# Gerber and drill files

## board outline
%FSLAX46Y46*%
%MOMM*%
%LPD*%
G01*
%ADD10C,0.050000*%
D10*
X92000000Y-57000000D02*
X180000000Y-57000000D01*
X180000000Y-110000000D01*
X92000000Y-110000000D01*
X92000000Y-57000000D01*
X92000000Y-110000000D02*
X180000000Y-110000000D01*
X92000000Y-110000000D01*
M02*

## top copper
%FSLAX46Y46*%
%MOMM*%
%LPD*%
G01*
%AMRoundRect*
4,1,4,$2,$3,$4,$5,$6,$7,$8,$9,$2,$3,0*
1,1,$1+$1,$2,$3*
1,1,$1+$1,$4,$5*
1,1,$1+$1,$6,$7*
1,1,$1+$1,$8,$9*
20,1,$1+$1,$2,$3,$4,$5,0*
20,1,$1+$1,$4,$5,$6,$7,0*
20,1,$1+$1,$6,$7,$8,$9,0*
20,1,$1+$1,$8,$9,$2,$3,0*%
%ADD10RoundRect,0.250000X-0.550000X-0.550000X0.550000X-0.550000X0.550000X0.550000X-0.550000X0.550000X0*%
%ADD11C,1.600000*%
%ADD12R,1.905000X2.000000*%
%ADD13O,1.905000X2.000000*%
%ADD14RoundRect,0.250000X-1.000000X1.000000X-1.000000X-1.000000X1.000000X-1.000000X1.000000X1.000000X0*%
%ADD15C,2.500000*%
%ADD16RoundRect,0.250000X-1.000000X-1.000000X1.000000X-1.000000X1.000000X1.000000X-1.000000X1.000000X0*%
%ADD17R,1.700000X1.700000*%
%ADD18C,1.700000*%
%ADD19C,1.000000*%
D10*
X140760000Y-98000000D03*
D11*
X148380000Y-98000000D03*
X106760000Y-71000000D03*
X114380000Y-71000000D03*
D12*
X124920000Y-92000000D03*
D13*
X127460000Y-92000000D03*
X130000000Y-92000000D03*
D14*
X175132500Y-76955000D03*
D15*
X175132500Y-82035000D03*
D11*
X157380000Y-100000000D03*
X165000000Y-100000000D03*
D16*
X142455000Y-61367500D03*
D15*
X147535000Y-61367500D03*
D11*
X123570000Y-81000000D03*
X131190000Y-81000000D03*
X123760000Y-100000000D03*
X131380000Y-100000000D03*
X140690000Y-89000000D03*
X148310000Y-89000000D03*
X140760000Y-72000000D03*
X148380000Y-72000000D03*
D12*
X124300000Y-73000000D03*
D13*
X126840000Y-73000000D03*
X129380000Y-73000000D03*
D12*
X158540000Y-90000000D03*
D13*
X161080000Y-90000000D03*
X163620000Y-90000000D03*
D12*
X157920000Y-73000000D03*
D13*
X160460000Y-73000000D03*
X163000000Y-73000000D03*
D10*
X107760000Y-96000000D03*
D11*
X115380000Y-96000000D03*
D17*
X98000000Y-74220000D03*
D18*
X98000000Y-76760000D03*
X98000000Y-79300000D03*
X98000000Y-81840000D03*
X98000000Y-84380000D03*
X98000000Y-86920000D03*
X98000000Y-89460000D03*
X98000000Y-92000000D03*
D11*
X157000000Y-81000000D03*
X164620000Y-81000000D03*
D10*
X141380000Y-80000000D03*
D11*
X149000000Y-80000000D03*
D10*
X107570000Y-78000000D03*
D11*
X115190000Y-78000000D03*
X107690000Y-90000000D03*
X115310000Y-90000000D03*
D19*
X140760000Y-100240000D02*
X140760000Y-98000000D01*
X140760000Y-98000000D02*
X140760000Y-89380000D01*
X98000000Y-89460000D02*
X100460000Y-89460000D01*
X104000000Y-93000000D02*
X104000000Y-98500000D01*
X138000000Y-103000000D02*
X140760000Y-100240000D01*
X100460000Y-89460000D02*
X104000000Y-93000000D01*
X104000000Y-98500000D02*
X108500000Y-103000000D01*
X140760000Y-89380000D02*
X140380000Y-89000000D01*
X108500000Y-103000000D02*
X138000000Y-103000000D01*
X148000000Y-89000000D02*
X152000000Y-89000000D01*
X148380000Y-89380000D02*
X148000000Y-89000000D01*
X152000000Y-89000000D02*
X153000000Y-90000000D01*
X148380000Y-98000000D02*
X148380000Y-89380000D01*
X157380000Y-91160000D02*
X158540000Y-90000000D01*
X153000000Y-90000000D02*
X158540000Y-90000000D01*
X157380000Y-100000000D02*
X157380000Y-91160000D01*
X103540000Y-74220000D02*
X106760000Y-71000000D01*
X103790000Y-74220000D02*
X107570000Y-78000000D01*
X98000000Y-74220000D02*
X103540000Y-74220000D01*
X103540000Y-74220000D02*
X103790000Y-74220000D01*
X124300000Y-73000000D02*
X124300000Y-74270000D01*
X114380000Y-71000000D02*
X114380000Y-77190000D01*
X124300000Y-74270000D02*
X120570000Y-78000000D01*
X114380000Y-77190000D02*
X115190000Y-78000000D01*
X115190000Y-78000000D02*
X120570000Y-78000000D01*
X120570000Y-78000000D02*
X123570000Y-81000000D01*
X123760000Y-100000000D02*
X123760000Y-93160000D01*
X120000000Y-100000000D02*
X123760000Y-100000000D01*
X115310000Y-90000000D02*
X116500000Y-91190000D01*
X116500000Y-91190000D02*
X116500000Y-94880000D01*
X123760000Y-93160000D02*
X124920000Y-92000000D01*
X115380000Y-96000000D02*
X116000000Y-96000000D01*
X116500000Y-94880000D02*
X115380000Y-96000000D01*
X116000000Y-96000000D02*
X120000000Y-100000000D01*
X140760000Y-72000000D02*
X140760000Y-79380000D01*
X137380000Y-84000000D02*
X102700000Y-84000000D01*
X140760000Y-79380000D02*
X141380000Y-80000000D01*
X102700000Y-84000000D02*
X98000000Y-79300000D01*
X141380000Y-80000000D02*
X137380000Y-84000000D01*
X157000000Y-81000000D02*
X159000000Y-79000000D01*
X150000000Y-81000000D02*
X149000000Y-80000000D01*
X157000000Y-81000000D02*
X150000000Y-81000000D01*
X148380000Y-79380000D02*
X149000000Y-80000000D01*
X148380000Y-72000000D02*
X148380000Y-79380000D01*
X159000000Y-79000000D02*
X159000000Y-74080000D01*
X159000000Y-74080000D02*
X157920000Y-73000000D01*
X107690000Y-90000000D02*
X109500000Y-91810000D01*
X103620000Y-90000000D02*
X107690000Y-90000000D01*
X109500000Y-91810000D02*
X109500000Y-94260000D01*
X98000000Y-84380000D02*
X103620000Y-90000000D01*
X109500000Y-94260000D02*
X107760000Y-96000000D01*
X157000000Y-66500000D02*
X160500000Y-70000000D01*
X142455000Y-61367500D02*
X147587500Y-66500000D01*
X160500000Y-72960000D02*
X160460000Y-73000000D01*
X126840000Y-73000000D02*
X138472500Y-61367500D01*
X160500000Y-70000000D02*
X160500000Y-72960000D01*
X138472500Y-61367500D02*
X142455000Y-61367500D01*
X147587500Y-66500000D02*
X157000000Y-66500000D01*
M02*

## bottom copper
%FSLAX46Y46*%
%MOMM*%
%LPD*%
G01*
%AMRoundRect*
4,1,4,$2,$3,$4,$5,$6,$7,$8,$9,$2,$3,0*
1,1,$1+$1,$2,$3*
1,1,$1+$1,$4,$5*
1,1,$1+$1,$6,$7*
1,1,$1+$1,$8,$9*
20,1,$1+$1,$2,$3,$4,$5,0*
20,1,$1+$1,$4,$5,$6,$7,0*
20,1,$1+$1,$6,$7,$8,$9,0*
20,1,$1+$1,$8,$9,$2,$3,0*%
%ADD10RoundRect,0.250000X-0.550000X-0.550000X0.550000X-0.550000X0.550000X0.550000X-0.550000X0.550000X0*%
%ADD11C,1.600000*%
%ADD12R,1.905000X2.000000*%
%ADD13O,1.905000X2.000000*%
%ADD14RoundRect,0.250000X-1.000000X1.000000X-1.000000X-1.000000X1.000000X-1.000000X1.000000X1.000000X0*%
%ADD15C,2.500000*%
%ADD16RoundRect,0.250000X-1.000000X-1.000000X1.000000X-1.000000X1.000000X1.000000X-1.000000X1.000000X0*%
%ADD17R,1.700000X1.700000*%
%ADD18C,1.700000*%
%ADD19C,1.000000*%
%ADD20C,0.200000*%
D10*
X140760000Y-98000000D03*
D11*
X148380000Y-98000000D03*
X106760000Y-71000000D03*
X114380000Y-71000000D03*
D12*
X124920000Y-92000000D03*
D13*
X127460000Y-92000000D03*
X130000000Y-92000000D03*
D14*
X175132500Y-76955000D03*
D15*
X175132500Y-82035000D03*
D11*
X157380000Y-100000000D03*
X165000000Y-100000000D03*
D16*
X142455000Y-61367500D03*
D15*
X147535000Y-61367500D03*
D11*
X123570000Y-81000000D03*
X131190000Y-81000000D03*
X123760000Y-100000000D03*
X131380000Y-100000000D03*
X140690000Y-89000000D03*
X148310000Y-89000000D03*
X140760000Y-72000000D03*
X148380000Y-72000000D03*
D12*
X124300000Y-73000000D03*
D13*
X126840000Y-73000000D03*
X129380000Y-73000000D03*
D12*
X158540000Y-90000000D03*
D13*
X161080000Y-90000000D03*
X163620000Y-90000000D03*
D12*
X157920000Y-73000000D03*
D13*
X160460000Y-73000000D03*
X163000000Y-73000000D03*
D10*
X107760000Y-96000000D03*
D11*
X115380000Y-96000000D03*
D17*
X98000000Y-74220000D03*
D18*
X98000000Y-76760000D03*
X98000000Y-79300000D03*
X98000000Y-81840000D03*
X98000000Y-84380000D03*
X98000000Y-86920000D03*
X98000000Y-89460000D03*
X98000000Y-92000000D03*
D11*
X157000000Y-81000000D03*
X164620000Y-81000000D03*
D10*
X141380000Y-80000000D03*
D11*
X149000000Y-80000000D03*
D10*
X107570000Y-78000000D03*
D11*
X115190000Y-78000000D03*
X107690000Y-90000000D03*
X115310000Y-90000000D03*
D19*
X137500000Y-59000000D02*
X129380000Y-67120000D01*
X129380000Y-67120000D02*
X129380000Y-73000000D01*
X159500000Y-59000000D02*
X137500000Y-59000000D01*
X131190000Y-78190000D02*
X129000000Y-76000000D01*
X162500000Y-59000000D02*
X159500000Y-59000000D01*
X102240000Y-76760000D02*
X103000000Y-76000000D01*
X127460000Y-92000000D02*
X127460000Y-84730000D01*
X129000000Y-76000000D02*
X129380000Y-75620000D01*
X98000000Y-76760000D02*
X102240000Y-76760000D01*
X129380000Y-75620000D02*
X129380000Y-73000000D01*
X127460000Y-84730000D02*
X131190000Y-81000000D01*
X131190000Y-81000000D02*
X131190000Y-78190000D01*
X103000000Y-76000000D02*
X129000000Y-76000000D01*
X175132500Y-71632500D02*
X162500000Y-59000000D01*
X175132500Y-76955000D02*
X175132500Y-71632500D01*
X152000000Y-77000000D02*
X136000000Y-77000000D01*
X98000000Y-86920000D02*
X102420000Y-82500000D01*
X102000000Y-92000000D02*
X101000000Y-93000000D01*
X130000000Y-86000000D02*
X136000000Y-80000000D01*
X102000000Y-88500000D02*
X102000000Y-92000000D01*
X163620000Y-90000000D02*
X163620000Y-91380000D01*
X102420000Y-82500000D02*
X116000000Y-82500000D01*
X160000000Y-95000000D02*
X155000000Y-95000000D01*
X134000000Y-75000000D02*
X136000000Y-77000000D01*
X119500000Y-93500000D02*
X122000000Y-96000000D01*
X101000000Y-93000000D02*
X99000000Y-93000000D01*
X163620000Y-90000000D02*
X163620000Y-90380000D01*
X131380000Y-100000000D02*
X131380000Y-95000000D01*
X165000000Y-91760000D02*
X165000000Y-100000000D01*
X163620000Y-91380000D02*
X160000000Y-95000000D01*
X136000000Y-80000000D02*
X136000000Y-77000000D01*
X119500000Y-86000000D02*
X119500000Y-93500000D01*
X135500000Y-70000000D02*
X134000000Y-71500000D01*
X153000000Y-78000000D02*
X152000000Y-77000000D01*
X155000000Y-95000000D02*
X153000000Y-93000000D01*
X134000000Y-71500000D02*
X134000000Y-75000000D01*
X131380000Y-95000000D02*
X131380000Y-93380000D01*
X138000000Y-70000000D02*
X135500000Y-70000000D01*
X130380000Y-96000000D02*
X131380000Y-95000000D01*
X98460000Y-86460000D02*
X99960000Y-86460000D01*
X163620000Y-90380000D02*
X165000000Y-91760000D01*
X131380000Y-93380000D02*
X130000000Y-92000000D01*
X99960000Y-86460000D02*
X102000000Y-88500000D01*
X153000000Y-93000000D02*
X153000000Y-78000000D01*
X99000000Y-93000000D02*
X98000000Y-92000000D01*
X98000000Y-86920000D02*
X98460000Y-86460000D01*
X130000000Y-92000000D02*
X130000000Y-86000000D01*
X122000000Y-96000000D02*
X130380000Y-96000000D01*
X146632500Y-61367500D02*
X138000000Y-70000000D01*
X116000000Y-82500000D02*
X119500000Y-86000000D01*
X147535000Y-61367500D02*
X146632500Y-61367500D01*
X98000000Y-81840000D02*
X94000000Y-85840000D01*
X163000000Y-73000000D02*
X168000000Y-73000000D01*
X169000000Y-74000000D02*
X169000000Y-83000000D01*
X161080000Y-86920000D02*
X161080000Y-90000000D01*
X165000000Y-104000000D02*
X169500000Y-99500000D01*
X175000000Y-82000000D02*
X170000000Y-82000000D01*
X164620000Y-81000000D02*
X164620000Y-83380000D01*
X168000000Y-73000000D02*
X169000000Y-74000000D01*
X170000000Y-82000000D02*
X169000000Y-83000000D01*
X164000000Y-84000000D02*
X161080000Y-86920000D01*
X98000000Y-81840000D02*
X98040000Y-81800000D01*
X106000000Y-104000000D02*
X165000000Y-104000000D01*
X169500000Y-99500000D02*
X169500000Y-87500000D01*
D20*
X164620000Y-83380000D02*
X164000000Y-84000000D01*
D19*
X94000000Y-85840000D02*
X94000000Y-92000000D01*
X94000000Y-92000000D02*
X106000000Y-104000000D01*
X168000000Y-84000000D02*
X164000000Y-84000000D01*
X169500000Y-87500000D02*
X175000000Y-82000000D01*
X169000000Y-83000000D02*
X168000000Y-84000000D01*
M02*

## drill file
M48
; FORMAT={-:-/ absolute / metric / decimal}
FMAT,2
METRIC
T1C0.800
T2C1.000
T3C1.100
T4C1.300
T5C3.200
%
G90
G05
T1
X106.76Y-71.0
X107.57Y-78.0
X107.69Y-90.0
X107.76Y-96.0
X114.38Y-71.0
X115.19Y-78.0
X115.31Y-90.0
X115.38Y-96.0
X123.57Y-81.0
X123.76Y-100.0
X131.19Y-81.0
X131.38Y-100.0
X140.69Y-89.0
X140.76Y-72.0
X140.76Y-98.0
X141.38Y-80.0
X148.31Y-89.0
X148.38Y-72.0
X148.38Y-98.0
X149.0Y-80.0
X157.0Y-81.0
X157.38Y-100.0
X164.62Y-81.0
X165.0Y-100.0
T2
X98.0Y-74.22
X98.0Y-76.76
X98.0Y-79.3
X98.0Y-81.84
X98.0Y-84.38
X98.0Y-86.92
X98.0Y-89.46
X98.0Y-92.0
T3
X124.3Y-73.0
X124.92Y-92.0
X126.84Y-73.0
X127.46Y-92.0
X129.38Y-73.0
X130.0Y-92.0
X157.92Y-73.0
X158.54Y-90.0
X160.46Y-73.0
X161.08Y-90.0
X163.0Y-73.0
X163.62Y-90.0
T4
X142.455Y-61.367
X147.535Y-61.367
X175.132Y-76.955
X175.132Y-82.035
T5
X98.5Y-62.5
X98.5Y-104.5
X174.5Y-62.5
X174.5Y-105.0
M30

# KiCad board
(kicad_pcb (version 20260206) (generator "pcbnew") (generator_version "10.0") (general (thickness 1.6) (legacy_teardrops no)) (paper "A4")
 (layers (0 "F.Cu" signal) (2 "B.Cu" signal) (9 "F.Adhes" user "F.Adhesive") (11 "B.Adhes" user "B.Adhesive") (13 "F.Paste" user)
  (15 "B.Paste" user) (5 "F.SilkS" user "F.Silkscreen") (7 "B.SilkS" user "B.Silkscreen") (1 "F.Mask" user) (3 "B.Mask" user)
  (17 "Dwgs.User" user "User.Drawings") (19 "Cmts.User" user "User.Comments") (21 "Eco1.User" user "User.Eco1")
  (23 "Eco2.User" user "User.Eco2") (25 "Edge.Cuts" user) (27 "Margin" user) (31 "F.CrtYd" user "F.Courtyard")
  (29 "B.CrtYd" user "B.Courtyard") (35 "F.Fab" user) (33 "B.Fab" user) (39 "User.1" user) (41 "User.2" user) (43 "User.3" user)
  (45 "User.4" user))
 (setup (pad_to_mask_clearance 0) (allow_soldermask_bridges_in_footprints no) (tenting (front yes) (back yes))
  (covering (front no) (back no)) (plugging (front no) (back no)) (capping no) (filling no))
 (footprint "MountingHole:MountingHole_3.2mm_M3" (layer "F.Cu") (at 98.5 62.5)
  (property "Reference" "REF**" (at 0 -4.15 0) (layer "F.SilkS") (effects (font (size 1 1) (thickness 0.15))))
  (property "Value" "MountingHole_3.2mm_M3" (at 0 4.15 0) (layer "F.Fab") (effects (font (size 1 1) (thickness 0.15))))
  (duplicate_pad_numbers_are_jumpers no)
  (pad "" np_thru_hole circle (at 0 0) (size 3.2 3.2) (drill 3.2) (layers "*.Cu" "*.Mask")))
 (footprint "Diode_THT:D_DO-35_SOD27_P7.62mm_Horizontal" (layer "F.Cu") (at 140.76 98)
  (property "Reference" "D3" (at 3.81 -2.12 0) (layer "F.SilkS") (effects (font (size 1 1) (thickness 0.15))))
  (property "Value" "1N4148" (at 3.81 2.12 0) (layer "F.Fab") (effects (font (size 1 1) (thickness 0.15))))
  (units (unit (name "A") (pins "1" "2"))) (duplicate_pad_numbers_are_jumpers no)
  (pad "1" thru_hole roundrect (at 0 0) (size 1.6 1.6) (drill 0.8) (layers "*.Cu" "*.Mask") (remove_unused_layers no)
   (roundrect_rratio 0.15625) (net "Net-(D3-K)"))
  (pad "2" thru_hole circle (at 7.62 0) (size 1.6 1.6) (drill 0.8) (layers "*.Cu" "*.Mask") (remove_unused_layers no) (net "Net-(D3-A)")))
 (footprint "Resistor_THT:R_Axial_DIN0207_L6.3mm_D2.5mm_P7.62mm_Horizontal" (layer "F.Cu") (at 106.76 71)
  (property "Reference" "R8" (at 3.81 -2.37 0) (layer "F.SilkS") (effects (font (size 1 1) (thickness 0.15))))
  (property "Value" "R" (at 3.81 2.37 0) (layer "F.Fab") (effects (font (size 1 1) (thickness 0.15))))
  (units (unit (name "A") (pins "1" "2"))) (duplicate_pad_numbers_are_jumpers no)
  (pad "1" thru_hole circle (at 0 0) (size 1.6 1.6) (drill 0.8) (layers "*.Cu" "*.Mask") (remove_unused_layers no) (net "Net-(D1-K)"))
  (pad "2" thru_hole circle (at 7.62 0) (size 1.6 1.6) (drill 0.8) (layers "*.Cu" "*.Mask") (remove_unused_layers no) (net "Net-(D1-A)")))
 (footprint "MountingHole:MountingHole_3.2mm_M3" (layer "F.Cu") (at 174.5 105)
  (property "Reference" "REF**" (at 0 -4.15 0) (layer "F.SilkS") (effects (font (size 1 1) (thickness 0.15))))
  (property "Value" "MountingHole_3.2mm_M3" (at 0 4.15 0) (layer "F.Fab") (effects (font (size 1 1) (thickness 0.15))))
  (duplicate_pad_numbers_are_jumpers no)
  (pad "" np_thru_hole circle (at 0 0) (size 3.2 3.2) (drill 3.2) (layers "*.Cu" "*.Mask")))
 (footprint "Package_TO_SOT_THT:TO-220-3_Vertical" (layer "F.Cu") (at 124.92 92)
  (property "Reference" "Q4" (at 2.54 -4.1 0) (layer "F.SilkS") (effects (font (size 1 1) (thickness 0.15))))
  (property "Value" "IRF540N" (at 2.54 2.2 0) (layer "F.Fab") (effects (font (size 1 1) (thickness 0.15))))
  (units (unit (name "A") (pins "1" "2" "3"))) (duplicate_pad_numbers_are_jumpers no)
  (pad "1" thru_hole rect (at 0 0) (size 1.905 2) (drill 1.1) (layers "*.Cu" "*.Mask") (remove_unused_layers no) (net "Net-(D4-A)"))
  (pad "2" thru_hole oval (at 2.54 0) (size 1.905 2) (drill 1.1) (layers "*.Cu" "*.Mask") (remove_unused_layers no) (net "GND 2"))
  (pad "3" thru_hole oval (at 5.08 0) (size 1.905 2) (drill 1.1) (layers "*.Cu" "*.Mask") (remove_unused_layers no) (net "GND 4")))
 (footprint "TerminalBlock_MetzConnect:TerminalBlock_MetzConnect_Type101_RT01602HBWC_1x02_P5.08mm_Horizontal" (layer "F.Cu")
  (at 175.1325 76.955 -90)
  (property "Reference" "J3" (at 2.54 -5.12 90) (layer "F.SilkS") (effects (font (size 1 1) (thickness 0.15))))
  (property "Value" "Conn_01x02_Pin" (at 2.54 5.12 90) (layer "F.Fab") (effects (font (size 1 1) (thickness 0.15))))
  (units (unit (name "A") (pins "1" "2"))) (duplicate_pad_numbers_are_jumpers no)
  (pad "1" thru_hole roundrect (at 0 0 270) (size 2.5 2.5) (drill 1.3) (layers "*.Cu" "*.Mask") (remove_unused_layers no)
   (roundrect_rratio 0.1) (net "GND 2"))
  (pad "2" thru_hole circle (at 5.08 0 270) (size 2.5 2.5) (drill 1.3) (layers "*.Cu" "*.Mask") (remove_unused_layers no) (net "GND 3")))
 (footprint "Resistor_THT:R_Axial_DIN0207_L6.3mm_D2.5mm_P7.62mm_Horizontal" (layer "F.Cu") (at 157.38 100)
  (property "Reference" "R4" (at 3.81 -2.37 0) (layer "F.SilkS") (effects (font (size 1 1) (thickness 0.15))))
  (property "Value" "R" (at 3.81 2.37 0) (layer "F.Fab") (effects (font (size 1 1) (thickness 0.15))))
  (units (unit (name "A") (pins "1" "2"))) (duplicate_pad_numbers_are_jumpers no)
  (pad "1" thru_hole circle (at 0 0) (size 1.6 1.6) (drill 0.8) (layers "*.Cu" "*.Mask") (remove_unused_layers no) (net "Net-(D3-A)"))
  (pad "2" thru_hole circle (at 7.62 0) (size 1.6 1.6) (drill 0.8) (layers "*.Cu" "*.Mask") (remove_unused_layers no) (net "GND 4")))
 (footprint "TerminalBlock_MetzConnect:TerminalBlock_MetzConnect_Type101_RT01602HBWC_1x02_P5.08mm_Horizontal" (layer "F.Cu")
  (at 142.455 61.3675)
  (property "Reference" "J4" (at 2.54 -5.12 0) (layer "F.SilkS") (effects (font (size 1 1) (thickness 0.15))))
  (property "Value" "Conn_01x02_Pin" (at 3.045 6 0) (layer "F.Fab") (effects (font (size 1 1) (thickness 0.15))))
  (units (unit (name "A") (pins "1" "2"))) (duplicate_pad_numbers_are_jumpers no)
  (pad "1" thru_hole roundrect (at 0 0) (size 2.5 2.5) (drill 1.3) (layers "*.Cu" "*.Mask") (remove_unused_layers no) (roundrect_rratio 0.1)
   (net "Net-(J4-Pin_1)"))
  (pad "2" thru_hole circle (at 5.08 0) (size 2.5 2.5) (drill 1.3) (layers "*.Cu" "*.Mask") (remove_unused_layers no) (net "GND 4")))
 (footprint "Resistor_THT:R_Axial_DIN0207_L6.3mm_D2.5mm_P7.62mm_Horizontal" (layer "F.Cu") (at 123.57 81)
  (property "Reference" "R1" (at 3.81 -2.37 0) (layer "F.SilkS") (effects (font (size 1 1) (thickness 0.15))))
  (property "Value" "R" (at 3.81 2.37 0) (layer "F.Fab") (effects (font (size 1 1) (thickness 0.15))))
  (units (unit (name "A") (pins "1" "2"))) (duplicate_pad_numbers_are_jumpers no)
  (pad "1" thru_hole circle (at 0 0) (size 1.6 1.6) (drill 0.8) (layers "*.Cu" "*.Mask") (remove_unused_layers no) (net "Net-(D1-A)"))
  (pad "2" thru_hole circle (at 7.62 0) (size 1.6 1.6) (drill 0.8) (layers "*.Cu" "*.Mask") (remove_unused_layers no) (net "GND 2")))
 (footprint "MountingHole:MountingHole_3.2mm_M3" (layer "F.Cu") (at 174.5 62.5)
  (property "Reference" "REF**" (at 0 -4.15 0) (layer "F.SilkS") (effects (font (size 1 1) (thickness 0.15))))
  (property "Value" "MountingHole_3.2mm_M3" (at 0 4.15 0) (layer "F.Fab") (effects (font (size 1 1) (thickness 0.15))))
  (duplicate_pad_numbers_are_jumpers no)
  (pad "" np_thru_hole circle (at 0 0) (size 3.2 3.2) (drill 3.2) (layers "*.Cu" "*.Mask")))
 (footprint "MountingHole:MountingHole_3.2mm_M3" (layer "F.Cu") (at 98.5 104.5)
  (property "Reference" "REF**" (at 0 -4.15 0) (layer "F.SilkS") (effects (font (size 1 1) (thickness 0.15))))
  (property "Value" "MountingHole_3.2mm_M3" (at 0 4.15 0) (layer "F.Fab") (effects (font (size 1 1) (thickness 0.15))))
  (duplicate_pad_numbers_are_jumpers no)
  (pad "" np_thru_hole circle (at 0 0) (size 3.2 3.2) (drill 3.2) (layers "*.Cu" "*.Mask")))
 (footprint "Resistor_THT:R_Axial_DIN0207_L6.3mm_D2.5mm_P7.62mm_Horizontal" (layer "F.Cu") (at 123.76 100)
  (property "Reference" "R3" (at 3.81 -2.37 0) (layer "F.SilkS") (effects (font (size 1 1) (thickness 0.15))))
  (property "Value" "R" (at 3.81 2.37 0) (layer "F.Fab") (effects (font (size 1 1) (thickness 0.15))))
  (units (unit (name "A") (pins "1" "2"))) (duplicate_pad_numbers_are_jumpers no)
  (pad "1" thru_hole circle (at 0 0) (size 1.6 1.6) (drill 0.8) (layers "*.Cu" "*.Mask") (remove_unused_layers no) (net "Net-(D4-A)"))
  (pad "2" thru_hole circle (at 7.62 0) (size 1.6 1.6) (drill 0.8) (layers "*.Cu" "*.Mask") (remove_unused_layers no) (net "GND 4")))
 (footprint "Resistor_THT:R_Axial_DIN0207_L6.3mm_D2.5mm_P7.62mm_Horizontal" (layer "F.Cu") (at 140.69 89)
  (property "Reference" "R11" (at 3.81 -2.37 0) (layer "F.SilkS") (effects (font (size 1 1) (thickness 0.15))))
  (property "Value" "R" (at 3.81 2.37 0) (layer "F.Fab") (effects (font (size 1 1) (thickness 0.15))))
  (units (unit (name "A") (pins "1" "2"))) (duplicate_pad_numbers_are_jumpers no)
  (pad "1" thru_hole circle (at 0 0) (size 1.6 1.6) (drill 0.8) (layers "*.Cu" "*.Mask") (remove_unused_layers no) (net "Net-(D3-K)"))
  (pad "2" thru_hole circle (at 7.62 0) (size 1.6 1.6) (drill 0.8) (layers "*.Cu" "*.Mask") (remove_unused_layers no) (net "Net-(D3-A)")))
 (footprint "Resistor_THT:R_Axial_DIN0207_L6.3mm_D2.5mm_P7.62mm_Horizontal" (layer "F.Cu") (at 140.76 72)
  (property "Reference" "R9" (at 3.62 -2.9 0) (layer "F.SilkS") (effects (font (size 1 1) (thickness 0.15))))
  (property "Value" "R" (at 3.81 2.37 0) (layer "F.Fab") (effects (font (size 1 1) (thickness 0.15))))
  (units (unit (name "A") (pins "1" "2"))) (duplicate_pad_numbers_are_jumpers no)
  (pad "1" thru_hole circle (at 0 0) (size 1.6 1.6) (drill 0.8) (layers "*.Cu" "*.Mask") (remove_unused_layers no) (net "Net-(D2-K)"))
  (pad "2" thru_hole circle (at 7.62 0) (size 1.6 1.6) (drill 0.8) (layers "*.Cu" "*.Mask") (remove_unused_layers no) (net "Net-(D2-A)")))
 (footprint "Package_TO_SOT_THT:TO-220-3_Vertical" (layer "F.Cu") (at 124.3 73)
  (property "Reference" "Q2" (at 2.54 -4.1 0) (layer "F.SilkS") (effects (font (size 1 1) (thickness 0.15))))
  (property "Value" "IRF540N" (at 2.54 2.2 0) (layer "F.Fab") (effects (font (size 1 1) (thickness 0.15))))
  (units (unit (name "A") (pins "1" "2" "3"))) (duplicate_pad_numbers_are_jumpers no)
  (pad "1" thru_hole rect (at 0 0) (size 1.905 2) (drill 1.1) (layers "*.Cu" "*.Mask") (remove_unused_layers no) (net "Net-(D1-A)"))
  (pad "2" thru_hole oval (at 2.54 0) (size 1.905 2) (drill 1.1) (layers "*.Cu" "*.Mask") (remove_unused_layers no) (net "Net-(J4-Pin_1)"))
  (pad "3" thru_hole oval (at 5.08 0) (size 1.905 2) (drill 1.1) (layers "*.Cu" "*.Mask") (remove_unused_layers no) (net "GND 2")))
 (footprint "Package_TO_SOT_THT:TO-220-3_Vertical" (layer "F.Cu") (at 158.54 90)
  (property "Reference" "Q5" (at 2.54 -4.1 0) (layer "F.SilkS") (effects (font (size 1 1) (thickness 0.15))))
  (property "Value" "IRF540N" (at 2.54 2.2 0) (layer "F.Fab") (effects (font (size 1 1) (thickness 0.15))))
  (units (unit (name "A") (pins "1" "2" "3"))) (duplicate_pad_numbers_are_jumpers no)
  (pad "1" thru_hole rect (at 0 0) (size 1.905 2) (drill 1.1) (layers "*.Cu" "*.Mask") (remove_unused_layers no) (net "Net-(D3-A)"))
  (pad "2" thru_hole oval (at 2.54 0) (size 1.905 2) (drill 1.1) (layers "*.Cu" "*.Mask") (remove_unused_layers no) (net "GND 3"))
  (pad "3" thru_hole oval (at 5.08 0) (size 1.905 2) (drill 1.1) (layers "*.Cu" "*.Mask") (remove_unused_layers no) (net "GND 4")))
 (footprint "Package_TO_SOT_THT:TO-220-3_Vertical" (layer "F.Cu") (at 157.92 73)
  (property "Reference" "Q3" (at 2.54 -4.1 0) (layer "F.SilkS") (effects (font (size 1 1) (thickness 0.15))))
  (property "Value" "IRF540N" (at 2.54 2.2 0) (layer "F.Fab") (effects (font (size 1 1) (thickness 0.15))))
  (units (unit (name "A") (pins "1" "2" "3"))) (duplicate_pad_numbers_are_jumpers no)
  (pad "1" thru_hole rect (at 0 0) (size 1.905 2) (drill 1.1) (layers "*.Cu" "*.Mask") (remove_unused_layers no) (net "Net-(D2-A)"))
  (pad "2" thru_hole oval (at 2.54 0) (size 1.905 2) (drill 1.1) (layers "*.Cu" "*.Mask") (remove_unused_layers no) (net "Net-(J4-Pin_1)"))
  (pad "3" thru_hole oval (at 5.08 0) (size 1.905 2) (drill 1.1) (layers "*.Cu" "*.Mask") (remove_unused_layers no) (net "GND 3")))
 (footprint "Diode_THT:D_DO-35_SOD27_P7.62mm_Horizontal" (layer "F.Cu") (at 107.76 96)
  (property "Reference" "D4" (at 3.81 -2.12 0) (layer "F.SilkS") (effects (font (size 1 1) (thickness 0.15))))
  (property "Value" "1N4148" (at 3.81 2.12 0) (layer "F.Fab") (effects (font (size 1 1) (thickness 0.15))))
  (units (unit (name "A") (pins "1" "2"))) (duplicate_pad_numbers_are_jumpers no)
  (pad "1" thru_hole roundrect (at 0 0) (size 1.6 1.6) (drill 0.8) (layers "*.Cu" "*.Mask") (remove_unused_layers no)
   (roundrect_rratio 0.15625) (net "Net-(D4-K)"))
  (pad "2" thru_hole circle (at 7.62 0) (size 1.6 1.6) (drill 0.8) (layers "*.Cu" "*.Mask") (remove_unused_layers no) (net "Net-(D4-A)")))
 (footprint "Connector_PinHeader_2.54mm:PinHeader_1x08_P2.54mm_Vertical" (layer "F.Cu") (at 98 74.22)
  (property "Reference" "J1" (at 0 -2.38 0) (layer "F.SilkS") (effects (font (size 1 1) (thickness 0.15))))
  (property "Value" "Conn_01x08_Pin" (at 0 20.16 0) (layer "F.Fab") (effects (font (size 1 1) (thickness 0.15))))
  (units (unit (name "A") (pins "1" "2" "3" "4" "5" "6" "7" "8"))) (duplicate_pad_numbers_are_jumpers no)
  (pad "1" thru_hole rect (at 0 0) (size 1.7 1.7) (drill 1) (layers "*.Cu" "*.Mask") (remove_unused_layers no) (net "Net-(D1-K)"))
  (pad "2" thru_hole circle (at 0 2.54) (size 1.7 1.7) (drill 1) (layers "*.Cu" "*.Mask") (remove_unused_layers no) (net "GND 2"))
  (pad "3" thru_hole circle (at 0 5.08) (size 1.7 1.7) (drill 1) (layers "*.Cu" "*.Mask") (remove_unused_layers no) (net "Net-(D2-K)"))
  (pad "4" thru_hole circle (at 0 7.62) (size 1.7 1.7) (drill 1) (layers "*.Cu" "*.Mask") (remove_unused_layers no) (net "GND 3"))
  (pad "5" thru_hole circle (at 0 10.16) (size 1.7 1.7) (drill 1) (layers "*.Cu" "*.Mask") (remove_unused_layers no) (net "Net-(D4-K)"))
  (pad "6" thru_hole circle (at 0 12.7) (size 1.7 1.7) (drill 1) (layers "*.Cu" "*.Mask") (remove_unused_layers no) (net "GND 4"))
  (pad "7" thru_hole circle (at 0 15.24) (size 1.7 1.7) (drill 1) (layers "*.Cu" "*.Mask") (remove_unused_layers no) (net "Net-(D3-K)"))
  (pad "8" thru_hole circle (at 0 17.78) (size 1.7 1.7) (drill 1) (layers "*.Cu" "*.Mask") (remove_unused_layers no) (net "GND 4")))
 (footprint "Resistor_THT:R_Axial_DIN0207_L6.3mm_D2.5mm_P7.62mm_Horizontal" (layer "F.Cu") (at 157 81)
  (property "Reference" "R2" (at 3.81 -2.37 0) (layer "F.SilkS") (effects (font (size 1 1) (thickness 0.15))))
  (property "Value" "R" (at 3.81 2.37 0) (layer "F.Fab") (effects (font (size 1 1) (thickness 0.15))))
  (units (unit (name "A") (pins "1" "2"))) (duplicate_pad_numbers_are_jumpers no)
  (pad "1" thru_hole circle (at 0 0) (size 1.6 1.6) (drill 0.8) (layers "*.Cu" "*.Mask") (remove_unused_layers no) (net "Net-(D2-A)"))
  (pad "2" thru_hole circle (at 7.62 0) (size 1.6 1.6) (drill 0.8) (layers "*.Cu" "*.Mask") (remove_unused_layers no) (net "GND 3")))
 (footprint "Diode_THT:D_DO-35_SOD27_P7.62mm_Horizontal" (layer "F.Cu") (at 141.38 80)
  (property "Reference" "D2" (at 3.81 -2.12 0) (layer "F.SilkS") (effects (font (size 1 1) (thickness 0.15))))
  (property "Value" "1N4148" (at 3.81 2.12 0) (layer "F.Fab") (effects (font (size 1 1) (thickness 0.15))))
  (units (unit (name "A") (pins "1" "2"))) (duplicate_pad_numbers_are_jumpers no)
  (pad "1" thru_hole roundrect (at 0 0) (size 1.6 1.6) (drill 0.8) (layers "*.Cu" "*.Mask") (remove_unused_layers no)
   (roundrect_rratio 0.15625) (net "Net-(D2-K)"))
  (pad "2" thru_hole circle (at 7.62 0) (size 1.6 1.6) (drill 0.8) (layers "*.Cu" "*.Mask") (remove_unused_layers no) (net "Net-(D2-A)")))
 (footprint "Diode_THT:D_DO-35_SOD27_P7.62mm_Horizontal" (layer "F.Cu") (at 107.57 78)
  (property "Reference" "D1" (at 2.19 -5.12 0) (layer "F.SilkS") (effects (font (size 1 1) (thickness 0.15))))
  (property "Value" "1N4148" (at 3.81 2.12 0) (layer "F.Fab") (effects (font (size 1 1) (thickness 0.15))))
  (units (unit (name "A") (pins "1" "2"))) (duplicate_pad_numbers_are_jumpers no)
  (pad "1" thru_hole roundrect (at 0 0) (size 1.6 1.6) (drill 0.8) (layers "*.Cu" "*.Mask") (remove_unused_layers no)
   (roundrect_rratio 0.15625) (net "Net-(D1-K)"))
  (pad "2" thru_hole circle (at 7.62 0) (size 1.6 1.6) (drill 0.8) (layers "*.Cu" "*.Mask") (remove_unused_layers no) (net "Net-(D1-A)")))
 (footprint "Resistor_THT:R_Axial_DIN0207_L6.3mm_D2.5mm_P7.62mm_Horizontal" (layer "F.Cu") (at 107.69 90)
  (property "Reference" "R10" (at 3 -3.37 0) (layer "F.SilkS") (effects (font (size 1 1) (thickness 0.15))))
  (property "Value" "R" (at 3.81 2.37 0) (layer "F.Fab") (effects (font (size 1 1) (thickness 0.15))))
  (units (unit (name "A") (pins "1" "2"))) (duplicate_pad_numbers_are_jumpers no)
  (pad "1" thru_hole circle (at 0 0) (size 1.6 1.6) (drill 0.8) (layers "*.Cu" "*.Mask") (remove_unused_layers no) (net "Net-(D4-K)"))
  (pad "2" thru_hole circle (at 7.62 0) (size 1.6 1.6) (drill 0.8) (layers "*.Cu" "*.Mask") (remove_unused_layers no) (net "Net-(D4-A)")))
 (gr_rect (start 92 57) (end 180 110) (stroke (width 0.05) (type default)) (fill no) (layer "Edge.Cuts"))
 (gr_rect (start 92 110) (end 180 110) (stroke (width 0.05) (type default)) (fill no) (layer "Edge.Cuts"))
 (segment (start 140.76 100.24) (end 140.76 98) (width 1) (layer "F.Cu") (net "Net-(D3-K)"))
 (segment (start 140.76 98) (end 140.76 89.38) (width 1) (layer "F.Cu") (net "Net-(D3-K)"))
 (segment (start 98 89.46) (end 100.46 89.46) (width 1) (layer "F.Cu") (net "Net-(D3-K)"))
 (segment (start 104 93) (end 104 98.5) (width 1) (layer "F.Cu") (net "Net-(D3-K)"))
 (segment (start 138 103) (end 140.76 100.24) (width 1) (layer "F.Cu") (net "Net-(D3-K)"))
 (segment (start 100.46 89.46) (end 104 93) (width 1) (layer "F.Cu") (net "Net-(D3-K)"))
 (segment (start 104 98.5) (end 108.5 103) (width 1) (layer "F.Cu") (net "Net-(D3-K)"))
 (segment (start 140.76 89.38) (end 140.38 89) (width 1) (layer "F.Cu") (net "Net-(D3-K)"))
 (segment (start 108.5 103) (end 138 103) (width 1) (layer "F.Cu") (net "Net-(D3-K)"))
 (segment (start 148 89) (end 152 89) (width 1) (layer "F.Cu") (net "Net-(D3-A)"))
 (segment (start 148.38 89.38) (end 148 89) (width 1) (layer "F.Cu") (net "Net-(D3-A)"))
 (segment (start 152 89) (end 153 90) (width 1) (layer "F.Cu") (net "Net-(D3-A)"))
 (segment (start 148.38 98) (end 148.38 89.38) (width 1) (layer "F.Cu") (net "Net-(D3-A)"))
 (segment (start 157.38 91.16) (end 158.54 90) (width 1) (layer "F.Cu") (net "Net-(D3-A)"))
 (segment (start 153 90) (end 158.54 90) (width 1) (layer "F.Cu") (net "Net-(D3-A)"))
 (segment (start 157.38 100) (end 157.38 91.16) (width 1) (layer "F.Cu") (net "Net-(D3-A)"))
 (segment (start 103.54 74.22) (end 106.76 71) (width 1) (layer "F.Cu") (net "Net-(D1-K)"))
 (segment (start 103.79 74.22) (end 107.57 78) (width 1) (layer "F.Cu") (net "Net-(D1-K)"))
 (segment (start 98 74.22) (end 103.54 74.22) (width 1) (layer "F.Cu") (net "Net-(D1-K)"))
 (segment (start 103.54 74.22) (end 103.79 74.22) (width 1) (layer "F.Cu") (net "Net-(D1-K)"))
 (segment (start 124.3 73) (end 124.3 74.27) (width 1) (layer "F.Cu") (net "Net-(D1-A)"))
 (segment (start 114.38 71) (end 114.38 77.19) (width 1) (layer "F.Cu") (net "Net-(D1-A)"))
 (segment (start 124.3 74.27) (end 120.57 78) (width 1) (layer "F.Cu") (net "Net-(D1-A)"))
 (segment (start 114.38 77.19) (end 115.19 78) (width 1) (layer "F.Cu") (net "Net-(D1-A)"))
 (segment (start 115.19 78) (end 120.57 78) (width 1) (layer "F.Cu") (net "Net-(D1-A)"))
 (segment (start 120.57 78) (end 123.57 81) (width 1) (layer "F.Cu") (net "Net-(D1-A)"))
 (segment (start 123.76 100) (end 123.76 93.16) (width 1) (layer "F.Cu") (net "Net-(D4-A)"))
 (segment (start 120 100) (end 123.76 100) (width 1) (layer "F.Cu") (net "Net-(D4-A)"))
 (segment (start 115.31 90) (end 116.5 91.19) (width 1) (layer "F.Cu") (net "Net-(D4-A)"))
 (segment (start 116.5 91.19) (end 116.5 94.88) (width 1) (layer "F.Cu") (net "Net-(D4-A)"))
 (segment (start 123.76 93.16) (end 124.92 92) (width 1) (layer "F.Cu") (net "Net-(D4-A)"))
 (segment (start 115.38 96) (end 116 96) (width 1) (layer "F.Cu") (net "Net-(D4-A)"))
 (segment (start 116.5 94.88) (end 115.38 96) (width 1) (layer "F.Cu") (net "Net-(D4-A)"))
 (segment (start 116 96) (end 120 100) (width 1) (layer "F.Cu") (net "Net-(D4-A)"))
 (segment (start 137.5 59) (end 129.38 67.12) (width 1) (layer "B.Cu") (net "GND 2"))
 (segment (start 129.38 67.12) (end 129.38 73) (width 1) (layer "B.Cu") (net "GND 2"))
 (segment (start 159.5 59) (end 137.5 59) (width 1) (layer "B.Cu") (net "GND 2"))
 (segment (start 131.19 78.19) (end 129 76) (width 1) (layer "B.Cu") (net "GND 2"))
 (segment (start 162.5 59) (end 159.5 59) (width 1) (layer "B.Cu") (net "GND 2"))
 (segment (start 102.24 76.76) (end 103 76) (width 1) (layer "B.Cu") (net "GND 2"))
 (segment (start 127.46 92) (end 127.46 84.73) (width 1) (layer "B.Cu") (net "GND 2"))
 (segment (start 129 76) (end 129.38 75.62) (width 1) (layer "B.Cu") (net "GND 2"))
 (segment (start 98 76.76) (end 102.24 76.76) (width 1) (layer "B.Cu") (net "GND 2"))
 (segment (start 129.38 75.62) (end 129.38 73) (width 1) (layer "B.Cu") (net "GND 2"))
 (segment (start 127.46 84.73) (end 131.19 81) (width 1) (layer "B.Cu") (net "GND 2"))
 (segment (start 131.19 81) (end 131.19 78.19) (width 1) (layer "B.Cu") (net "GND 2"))
 (segment (start 103 76) (end 129 76) (width 1) (layer "B.Cu") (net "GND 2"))
 (segment (start 175.1325 71.6325) (end 162.5 59) (width 1) (layer "B.Cu") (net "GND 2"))
 (segment (start 175.1325 76.955) (end 175.1325 71.6325) (width 1) (layer "B.Cu") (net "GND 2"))
 (segment (start 152 77) (end 136 77) (width 1) (layer "B.Cu") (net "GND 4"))
 (segment (start 98 86.92) (end 102.42 82.5) (width 1) (layer "B.Cu") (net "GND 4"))
 (segment (start 102 92) (end 101 93) (width 1) (layer "B.Cu") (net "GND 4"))
 (segment (start 130 86) (end 136 80) (width 1) (layer "B.Cu") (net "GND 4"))
 (segment (start 102 88.5) (end 102 92) (width 1) (layer "B.Cu") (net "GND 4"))
 (segment (start 163.62 90) (end 163.62 91.38) (width 1) (layer "B.Cu") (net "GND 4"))
 (segment (start 102.42 82.5) (end 116 82.5) (width 1) (layer "B.Cu") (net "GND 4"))
 (segment (start 160 95) (end 155 95) (width 1) (layer "B.Cu") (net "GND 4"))
 (segment (start 134 75) (end 136 77) (width 1) (layer "B.Cu") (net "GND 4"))
 (segment (start 119.5 93.5) (end 122 96) (width 1) (layer "B.Cu") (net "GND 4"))
 (segment (start 101 93) (end 99 93) (width 1) (layer "B.Cu") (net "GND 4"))
 (segment (start 163.62 90) (end 163.62 90.38) (width 1) (layer "B.Cu") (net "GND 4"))
 (segment (start 131.38 100) (end 131.38 95) (width 1) (layer "B.Cu") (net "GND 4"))
 (segment (start 165 91.76) (end 165 100) (width 1) (layer "B.Cu") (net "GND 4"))
 (segment (start 163.62 91.38) (end 160 95) (width 1) (layer "B.Cu") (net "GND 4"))
 (segment (start 136 80) (end 136 77) (width 1) (layer "B.Cu") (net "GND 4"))
 (segment (start 119.5 86) (end 119.5 93.5) (width 1) (layer "B.Cu") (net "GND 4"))
 (segment (start 135.5 70) (end 134 71.5) (width 1) (layer "B.Cu") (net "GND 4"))
 (segment (start 153 78) (end 152 77) (width 1) (layer "B.Cu") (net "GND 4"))
 (segment (start 155 95) (end 153 93) (width 1) (layer "B.Cu") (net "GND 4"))
 (segment (start 134 71.5) (end 134 75) (width 1) (layer "B.Cu") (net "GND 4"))
 (segment (start 131.38 95) (end 131.38 93.38) (width 1) (layer "B.Cu") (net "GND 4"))
 (segment (start 138 70) (end 135.5 70) (width 1) (layer "B.Cu") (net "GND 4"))
 (segment (start 130.38 96) (end 131.38 95) (width 1) (layer "B.Cu") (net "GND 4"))
 (segment (start 98.46 86.46) (end 99.96 86.46) (width 1) (layer "B.Cu") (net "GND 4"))
 (segment (start 163.62 90.38) (end 165 91.76) (width 1) (layer "B.Cu") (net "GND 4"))
 (segment (start 131.38 93.38) (end 130 92) (width 1) (layer "B.Cu") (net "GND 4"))
 (segment (start 99.96 86.46) (end 102 88.5) (width 1) (layer "B.Cu") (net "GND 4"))
 (segment (start 153 93) (end 153 78) (width 1) (layer "B.Cu") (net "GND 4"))
 (segment (start 99 93) (end 98 92) (width 1) (layer "B.Cu") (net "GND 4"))
 (segment (start 98 86.92) (end 98.46 86.46) (width 1) (layer "B.Cu") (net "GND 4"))
 (segment (start 130 92) (end 130 86) (width 1) (layer "B.Cu") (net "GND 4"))
 (segment (start 122 96) (end 130.38 96) (width 1) (layer "B.Cu") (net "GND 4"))
 (segment (start 146.6325 61.3675) (end 138 70) (width 1) (layer "B.Cu") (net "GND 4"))
 (segment (start 116 82.5) (end 119.5 86) (width 1) (layer "B.Cu") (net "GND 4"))
 (segment (start 147.535 61.3675) (end 146.6325 61.3675) (width 1) (layer "B.Cu") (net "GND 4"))
 (segment (start 98 81.84) (end 94 85.84) (width 1) (layer "B.Cu") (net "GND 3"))
 (segment (start 163 73) (end 168 73) (width 1) (layer "B.Cu") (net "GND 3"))
 (segment (start 169 74) (end 169 83) (width 1) (layer "B.Cu") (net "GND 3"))
 (segment (start 161.08 86.92) (end 161.08 90) (width 1) (layer "B.Cu") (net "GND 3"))
 (segment (start 165 104) (end 169.5 99.5) (width 1) (layer "B.Cu") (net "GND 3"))
 (segment (start 175 82) (end 170 82) (width 1) (layer "B.Cu") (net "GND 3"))
 (segment (start 164.62 81) (end 164.62 83.38) (width 1) (layer "B.Cu") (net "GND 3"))
 (segment (start 168 73) (end 169 74) (width 1) (layer "B.Cu") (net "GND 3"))
 (segment (start 170 82) (end 169 83) (width 1) (layer "B.Cu") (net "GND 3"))
 (segment (start 164 84) (end 161.08 86.92) (width 1) (layer "B.Cu") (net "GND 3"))
 (segment (start 98 81.84) (end 98.04 81.8) (width 1) (layer "B.Cu") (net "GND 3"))
 (segment (start 106 104) (end 165 104) (width 1) (layer "B.Cu") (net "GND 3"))
 (segment (start 169.5 99.5) (end 169.5 87.5) (width 1) (layer "B.Cu") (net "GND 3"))
 (segment (start 164.62 83.38) (end 164 84) (width 0.2) (layer "B.Cu") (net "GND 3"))
 (segment (start 94 85.84) (end 94 92) (width 1) (layer "B.Cu") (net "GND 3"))
 (segment (start 94 92) (end 106 104) (width 1) (layer "B.Cu") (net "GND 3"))
 (segment (start 168 84) (end 164 84) (width 1) (layer "B.Cu") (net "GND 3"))
 (segment (start 169.5 87.5) (end 175 82) (width 1) (layer "B.Cu") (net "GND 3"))
 (segment (start 169 83) (end 168 84) (width 1) (layer "B.Cu") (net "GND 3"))
 (segment (start 140.76 72) (end 140.76 79.38) (width 1) (layer "F.Cu") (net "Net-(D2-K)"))
 (segment (start 137.38 84) (end 102.7 84) (width 1) (layer "F.Cu") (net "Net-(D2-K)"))
 (segment (start 140.76 79.38) (end 141.38 80) (width 1) (layer "F.Cu") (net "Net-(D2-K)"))
 (segment (start 102.7 84) (end 98 79.3) (width 1) (layer "F.Cu") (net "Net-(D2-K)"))
 (segment (start 141.38 80) (end 137.38 84) (width 1) (layer "F.Cu") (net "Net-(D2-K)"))
 (segment (start 157 81) (end 159 79) (width 1) (layer "F.Cu") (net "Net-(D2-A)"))
 (segment (start 150 81) (end 149 80) (width 1) (layer "F.Cu") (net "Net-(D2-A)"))
 (segment (start 157 81) (end 150 81) (width 1) (layer "F.Cu") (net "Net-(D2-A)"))
 (segment (start 148.38 79.38) (end 149 80) (width 1) (layer "F.Cu") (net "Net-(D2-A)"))
 (segment (start 148.38 72) (end 148.38 79.38) (width 1) (layer "F.Cu") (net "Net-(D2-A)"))
 (segment (start 159 79) (end 159 74.08) (width 1) (layer "F.Cu") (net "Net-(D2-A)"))
 (segment (start 159 74.08) (end 157.92 73) (width 1) (layer "F.Cu") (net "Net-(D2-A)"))
 (segment (start 107.69 90) (end 109.5 91.81) (width 1) (layer "F.Cu") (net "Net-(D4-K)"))
 (segment (start 103.62 90) (end 107.69 90) (width 1) (layer "F.Cu") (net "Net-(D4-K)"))
 (segment (start 109.5 91.81) (end 109.5 94.26) (width 1) (layer "F.Cu") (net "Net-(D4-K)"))
 (segment (start 98 84.38) (end 103.62 90) (width 1) (layer "F.Cu") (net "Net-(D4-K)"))
 (segment (start 109.5 94.26) (end 107.76 96) (width 1) (layer "F.Cu") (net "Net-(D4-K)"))
 (segment (start 157 66.5) (end 160.5 70) (width 1) (layer "F.Cu") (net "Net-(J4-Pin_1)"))
 (segment (start 142.455 61.3675) (end 147.5875 66.5) (width 1) (layer "F.Cu") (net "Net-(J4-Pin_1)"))
 (segment (start 160.5 72.96) (end 160.46 73) (width 1) (layer "F.Cu") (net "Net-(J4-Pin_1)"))
 (segment (start 126.84 73) (end 138.4725 61.3675) (width 1) (layer "F.Cu") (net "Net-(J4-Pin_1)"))
 (segment (start 160.5 70) (end 160.5 72.96) (width 1) (layer "F.Cu") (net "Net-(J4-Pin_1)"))
 (segment (start 138.4725 61.3675) (end 142.455 61.3675) (width 1) (layer "F.Cu") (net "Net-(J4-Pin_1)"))
 (segment (start 147.5875 66.5) (end 157 66.5) (width 1) (layer "F.Cu") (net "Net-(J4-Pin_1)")))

